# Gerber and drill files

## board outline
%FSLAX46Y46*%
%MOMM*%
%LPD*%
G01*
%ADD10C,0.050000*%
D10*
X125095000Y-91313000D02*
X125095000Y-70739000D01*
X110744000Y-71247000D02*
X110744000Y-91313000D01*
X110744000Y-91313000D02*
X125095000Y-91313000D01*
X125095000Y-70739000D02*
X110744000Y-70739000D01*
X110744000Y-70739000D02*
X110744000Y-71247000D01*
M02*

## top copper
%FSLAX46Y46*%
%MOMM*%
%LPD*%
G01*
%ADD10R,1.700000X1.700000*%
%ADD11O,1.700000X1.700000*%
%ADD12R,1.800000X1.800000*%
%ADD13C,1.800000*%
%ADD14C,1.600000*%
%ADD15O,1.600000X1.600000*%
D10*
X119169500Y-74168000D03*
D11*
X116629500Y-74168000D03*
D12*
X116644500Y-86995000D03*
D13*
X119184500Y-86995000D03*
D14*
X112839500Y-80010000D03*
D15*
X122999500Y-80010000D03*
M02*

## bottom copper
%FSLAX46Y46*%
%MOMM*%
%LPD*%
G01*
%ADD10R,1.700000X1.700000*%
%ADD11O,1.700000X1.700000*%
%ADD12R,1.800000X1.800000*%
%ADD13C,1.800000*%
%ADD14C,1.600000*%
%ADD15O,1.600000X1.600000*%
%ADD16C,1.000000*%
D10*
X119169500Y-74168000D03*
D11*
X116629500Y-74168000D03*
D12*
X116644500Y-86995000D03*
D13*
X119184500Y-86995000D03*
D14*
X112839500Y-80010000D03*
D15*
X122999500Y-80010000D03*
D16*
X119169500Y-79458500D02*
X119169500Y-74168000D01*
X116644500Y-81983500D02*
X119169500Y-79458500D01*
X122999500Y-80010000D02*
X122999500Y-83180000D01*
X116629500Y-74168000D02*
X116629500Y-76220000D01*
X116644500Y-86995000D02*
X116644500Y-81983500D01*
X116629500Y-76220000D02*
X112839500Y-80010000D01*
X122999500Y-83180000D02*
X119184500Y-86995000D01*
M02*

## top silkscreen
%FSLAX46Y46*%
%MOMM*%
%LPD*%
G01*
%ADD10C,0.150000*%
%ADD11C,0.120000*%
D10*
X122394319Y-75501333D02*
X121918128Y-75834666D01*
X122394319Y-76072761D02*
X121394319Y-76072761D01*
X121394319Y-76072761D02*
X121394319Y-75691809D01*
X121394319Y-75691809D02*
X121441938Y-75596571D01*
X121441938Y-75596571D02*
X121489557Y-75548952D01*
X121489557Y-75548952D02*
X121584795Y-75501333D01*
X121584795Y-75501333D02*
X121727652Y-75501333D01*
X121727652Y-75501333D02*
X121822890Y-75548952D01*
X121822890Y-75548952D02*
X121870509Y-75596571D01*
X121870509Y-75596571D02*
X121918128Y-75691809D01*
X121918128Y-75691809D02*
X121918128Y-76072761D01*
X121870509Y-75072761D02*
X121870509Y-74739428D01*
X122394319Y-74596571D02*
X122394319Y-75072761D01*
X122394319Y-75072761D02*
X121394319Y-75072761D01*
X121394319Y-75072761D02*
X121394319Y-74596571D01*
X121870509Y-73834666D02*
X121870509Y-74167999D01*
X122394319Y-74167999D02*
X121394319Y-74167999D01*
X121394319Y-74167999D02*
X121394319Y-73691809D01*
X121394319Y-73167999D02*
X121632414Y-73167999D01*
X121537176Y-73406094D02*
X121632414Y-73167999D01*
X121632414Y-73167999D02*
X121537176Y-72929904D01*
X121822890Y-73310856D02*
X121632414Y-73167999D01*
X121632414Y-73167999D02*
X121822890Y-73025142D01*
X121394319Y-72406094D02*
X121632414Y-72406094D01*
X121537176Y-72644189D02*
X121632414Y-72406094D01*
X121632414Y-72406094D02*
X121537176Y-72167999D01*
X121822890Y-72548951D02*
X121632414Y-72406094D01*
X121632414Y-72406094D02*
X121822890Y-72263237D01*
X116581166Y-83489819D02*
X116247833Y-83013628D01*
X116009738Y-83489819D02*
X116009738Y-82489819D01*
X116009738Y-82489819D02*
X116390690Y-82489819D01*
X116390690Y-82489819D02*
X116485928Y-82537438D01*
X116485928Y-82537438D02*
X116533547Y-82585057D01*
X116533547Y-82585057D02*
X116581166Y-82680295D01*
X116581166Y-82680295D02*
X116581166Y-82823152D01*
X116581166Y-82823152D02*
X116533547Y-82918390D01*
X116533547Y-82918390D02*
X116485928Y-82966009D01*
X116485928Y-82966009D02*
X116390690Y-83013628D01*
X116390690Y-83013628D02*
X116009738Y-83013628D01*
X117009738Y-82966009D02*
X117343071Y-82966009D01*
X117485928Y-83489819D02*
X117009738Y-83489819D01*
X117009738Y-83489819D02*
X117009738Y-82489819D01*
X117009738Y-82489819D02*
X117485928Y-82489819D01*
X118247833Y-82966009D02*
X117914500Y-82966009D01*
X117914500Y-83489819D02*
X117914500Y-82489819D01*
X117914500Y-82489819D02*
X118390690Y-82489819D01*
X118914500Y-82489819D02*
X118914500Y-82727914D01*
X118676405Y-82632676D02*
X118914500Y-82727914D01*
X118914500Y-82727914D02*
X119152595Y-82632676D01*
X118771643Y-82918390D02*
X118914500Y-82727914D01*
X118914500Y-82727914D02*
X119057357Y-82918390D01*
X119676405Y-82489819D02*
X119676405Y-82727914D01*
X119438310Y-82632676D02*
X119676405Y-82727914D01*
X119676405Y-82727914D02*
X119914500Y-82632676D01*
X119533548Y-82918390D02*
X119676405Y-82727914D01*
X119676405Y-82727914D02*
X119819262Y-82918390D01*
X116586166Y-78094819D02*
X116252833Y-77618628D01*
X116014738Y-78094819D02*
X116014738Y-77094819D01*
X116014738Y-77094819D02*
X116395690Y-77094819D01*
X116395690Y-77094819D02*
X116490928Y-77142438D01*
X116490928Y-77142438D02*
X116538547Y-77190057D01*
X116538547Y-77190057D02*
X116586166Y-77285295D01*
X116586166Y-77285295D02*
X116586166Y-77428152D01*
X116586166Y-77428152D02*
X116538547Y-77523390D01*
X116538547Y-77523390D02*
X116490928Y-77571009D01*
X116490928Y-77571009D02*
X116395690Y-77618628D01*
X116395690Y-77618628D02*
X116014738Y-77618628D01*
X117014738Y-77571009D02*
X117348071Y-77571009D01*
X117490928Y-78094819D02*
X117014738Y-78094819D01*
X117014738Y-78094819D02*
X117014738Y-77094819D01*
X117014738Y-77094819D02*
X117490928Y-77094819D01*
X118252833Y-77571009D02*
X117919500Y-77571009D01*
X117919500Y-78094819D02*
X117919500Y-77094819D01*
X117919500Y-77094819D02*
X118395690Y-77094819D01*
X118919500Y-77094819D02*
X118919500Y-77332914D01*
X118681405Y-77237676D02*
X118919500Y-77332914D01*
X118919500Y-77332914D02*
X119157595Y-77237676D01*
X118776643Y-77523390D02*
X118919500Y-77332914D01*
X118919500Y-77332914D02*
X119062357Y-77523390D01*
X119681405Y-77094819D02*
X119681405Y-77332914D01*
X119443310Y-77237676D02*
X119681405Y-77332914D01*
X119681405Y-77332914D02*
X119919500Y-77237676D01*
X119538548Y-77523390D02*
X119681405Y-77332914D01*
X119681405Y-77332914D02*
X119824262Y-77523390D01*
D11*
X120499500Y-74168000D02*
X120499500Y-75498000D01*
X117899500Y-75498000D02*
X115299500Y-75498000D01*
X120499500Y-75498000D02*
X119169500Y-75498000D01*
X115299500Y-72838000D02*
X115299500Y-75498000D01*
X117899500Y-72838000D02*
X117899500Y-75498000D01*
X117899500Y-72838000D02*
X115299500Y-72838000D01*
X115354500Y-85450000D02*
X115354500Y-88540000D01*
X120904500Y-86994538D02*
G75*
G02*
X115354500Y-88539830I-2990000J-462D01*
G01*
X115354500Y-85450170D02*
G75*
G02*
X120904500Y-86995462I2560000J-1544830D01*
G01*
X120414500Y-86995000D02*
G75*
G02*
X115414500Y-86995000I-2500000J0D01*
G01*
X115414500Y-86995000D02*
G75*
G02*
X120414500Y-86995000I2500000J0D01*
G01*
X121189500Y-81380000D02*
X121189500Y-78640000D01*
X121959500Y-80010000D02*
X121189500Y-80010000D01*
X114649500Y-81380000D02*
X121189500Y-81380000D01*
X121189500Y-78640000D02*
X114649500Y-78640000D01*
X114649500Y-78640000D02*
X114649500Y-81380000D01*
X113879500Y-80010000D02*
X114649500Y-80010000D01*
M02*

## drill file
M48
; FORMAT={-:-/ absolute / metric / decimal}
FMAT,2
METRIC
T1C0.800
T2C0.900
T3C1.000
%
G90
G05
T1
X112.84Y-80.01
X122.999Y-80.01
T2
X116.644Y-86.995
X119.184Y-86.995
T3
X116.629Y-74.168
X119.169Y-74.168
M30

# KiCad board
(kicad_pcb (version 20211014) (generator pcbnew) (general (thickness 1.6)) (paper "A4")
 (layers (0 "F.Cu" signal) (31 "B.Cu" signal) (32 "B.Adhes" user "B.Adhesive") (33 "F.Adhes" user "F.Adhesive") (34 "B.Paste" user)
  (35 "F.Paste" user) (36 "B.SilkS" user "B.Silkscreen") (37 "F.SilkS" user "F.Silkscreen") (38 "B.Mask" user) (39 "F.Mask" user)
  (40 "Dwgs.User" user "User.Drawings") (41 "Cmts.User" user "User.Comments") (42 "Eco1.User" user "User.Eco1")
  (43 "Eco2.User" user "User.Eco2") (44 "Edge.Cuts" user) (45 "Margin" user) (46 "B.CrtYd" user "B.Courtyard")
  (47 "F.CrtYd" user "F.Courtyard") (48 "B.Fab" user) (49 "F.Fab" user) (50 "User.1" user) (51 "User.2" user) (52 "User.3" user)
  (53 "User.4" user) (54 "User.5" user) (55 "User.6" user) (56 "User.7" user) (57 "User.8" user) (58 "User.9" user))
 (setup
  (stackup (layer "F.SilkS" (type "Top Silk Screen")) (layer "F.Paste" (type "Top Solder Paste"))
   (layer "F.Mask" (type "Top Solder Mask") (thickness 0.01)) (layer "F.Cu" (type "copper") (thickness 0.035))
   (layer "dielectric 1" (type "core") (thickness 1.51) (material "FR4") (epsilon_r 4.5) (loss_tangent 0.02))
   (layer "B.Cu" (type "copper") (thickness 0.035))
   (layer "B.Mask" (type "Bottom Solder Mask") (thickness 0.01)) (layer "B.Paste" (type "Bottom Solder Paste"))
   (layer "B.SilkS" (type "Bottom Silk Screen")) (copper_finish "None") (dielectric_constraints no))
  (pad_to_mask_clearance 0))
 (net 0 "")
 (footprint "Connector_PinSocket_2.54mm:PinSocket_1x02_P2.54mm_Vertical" (layer "F.Cu") (at 119.1695 74.168 -90)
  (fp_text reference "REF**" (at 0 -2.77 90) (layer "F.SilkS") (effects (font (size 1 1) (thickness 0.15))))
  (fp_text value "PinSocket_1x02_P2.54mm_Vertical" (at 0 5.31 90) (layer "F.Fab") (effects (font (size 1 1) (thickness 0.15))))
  (fp_line (start 0 -1.33) (end 1.33 -1.33) (layer "F.SilkS") (width 0.12))
  (fp_line (start 1.33 1.27) (end 1.33 3.87) (layer "F.SilkS") (width 0.12))
  (fp_line (start 1.33 -1.33) (end 1.33 0) (layer "F.SilkS") (width 0.12))
  (fp_line (start -1.33 3.87) (end 1.33 3.87) (layer "F.SilkS") (width 0.12))
  (fp_line (start -1.33 1.27) (end 1.33 1.27) (layer "F.SilkS") (width 0.12))
  (fp_line (start -1.33 1.27) (end -1.33 3.87) (layer "F.SilkS") (width 0.12))
  (pad "1" thru_hole rect (at 0 0 270) (size 1.7 1.7) (drill 1) (layers *.Cu *.Mask))
  (pad "2" thru_hole oval (at 0 2.54 270) (size 1.7 1.7) (drill 1) (layers *.Cu *.Mask)))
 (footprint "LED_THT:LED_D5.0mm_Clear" (layer "F.Cu") (at 116.6445 86.995)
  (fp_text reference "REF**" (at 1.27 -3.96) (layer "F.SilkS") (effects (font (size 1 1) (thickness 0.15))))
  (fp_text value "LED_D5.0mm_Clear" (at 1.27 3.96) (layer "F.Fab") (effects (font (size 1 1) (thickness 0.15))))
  (fp_line (start -1.29 -1.545) (end -1.29 1.545) (layer "F.SilkS") (width 0.12))
  (fp_arc (start 4.26 -0.000462) (mid 2.072002 2.880433) (end -1.29 1.54483) (layer "F.SilkS") (width 0.12))
  (fp_arc (start -1.29 -1.54483) (mid 2.072002 -2.880433) (end 4.26 0.000462) (layer "F.SilkS") (width 0.12))
  (fp_circle (center 1.27 0) (end 3.77 0) (layer "F.SilkS") (width 0.12) (fill none))
  (pad "1" thru_hole rect (at 0 0) (size 1.8 1.8) (drill 0.9) (layers *.Cu *.Mask))
  (pad "2" thru_hole circle (at 2.54 0) (size 1.8 1.8) (drill 0.9) (layers *.Cu *.Mask)))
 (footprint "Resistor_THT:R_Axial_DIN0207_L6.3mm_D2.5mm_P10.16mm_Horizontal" (layer "F.Cu") (at 112.8395 80.01)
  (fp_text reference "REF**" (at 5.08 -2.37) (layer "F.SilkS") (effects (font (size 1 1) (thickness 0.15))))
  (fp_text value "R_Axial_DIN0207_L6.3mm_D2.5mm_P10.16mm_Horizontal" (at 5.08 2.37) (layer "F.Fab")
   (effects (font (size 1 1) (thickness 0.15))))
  (fp_line (start 8.35 1.37) (end 8.35 -1.37) (layer "F.SilkS") (width 0.12))
  (fp_line (start 9.12 0) (end 8.35 0) (layer "F.SilkS") (width 0.12))
  (fp_line (start 1.81 1.37) (end 8.35 1.37) (layer "F.SilkS") (width 0.12))
  (fp_line (start 8.35 -1.37) (end 1.81 -1.37) (layer "F.SilkS") (width 0.12))
  (fp_line (start 1.81 -1.37) (end 1.81 1.37) (layer "F.SilkS") (width 0.12))
  (fp_line (start 1.04 0) (end 1.81 0) (layer "F.SilkS") (width 0.12))
  (pad "1" thru_hole circle (at 0 0) (size 1.6 1.6) (drill 0.8) (layers *.Cu *.Mask))
  (pad "2" thru_hole oval (at 10.16 0) (size 1.6 1.6) (drill 0.8) (layers *.Cu *.Mask)))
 (gr_line (start 125.095 91.313) (end 125.095 70.739) (layer "Edge.Cuts") (width 0.05))
 (gr_line (start 110.744 71.247) (end 110.744 91.313) (layer "Edge.Cuts") (width 0.05))
 (gr_line (start 110.744 91.313) (end 125.095 91.313) (layer "Edge.Cuts") (width 0.05))
 (gr_line (start 125.095 70.739) (end 110.744 70.739) (layer "Edge.Cuts") (width 0.05))
 (gr_line (start 110.744 70.739) (end 110.744 71.247) (layer "Edge.Cuts") (width 0.05))
 (segment (start 119.1695 79.4585) (end 119.1695 74.168) (width 1) (layer "B.Cu") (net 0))
 (segment (start 116.6445 81.9835) (end 119.1695 79.4585) (width 1) (layer "B.Cu") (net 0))
 (segment (start 122.9995 80.01) (end 122.9995 83.18) (width 1) (layer "B.Cu") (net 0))
 (segment (start 116.6295 74.168) (end 116.6295 76.22) (width 1) (layer "B.Cu") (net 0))
 (segment (start 116.6445 86.995) (end 116.6445 81.9835) (width 1) (layer "B.Cu") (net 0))
 (segment (start 116.6295 76.22) (end 112.8395 80.01) (width 1) (layer "B.Cu") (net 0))
 (segment (start 122.9995 83.18) (end 119.1845 86.995) (width 1) (layer "B.Cu") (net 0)))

